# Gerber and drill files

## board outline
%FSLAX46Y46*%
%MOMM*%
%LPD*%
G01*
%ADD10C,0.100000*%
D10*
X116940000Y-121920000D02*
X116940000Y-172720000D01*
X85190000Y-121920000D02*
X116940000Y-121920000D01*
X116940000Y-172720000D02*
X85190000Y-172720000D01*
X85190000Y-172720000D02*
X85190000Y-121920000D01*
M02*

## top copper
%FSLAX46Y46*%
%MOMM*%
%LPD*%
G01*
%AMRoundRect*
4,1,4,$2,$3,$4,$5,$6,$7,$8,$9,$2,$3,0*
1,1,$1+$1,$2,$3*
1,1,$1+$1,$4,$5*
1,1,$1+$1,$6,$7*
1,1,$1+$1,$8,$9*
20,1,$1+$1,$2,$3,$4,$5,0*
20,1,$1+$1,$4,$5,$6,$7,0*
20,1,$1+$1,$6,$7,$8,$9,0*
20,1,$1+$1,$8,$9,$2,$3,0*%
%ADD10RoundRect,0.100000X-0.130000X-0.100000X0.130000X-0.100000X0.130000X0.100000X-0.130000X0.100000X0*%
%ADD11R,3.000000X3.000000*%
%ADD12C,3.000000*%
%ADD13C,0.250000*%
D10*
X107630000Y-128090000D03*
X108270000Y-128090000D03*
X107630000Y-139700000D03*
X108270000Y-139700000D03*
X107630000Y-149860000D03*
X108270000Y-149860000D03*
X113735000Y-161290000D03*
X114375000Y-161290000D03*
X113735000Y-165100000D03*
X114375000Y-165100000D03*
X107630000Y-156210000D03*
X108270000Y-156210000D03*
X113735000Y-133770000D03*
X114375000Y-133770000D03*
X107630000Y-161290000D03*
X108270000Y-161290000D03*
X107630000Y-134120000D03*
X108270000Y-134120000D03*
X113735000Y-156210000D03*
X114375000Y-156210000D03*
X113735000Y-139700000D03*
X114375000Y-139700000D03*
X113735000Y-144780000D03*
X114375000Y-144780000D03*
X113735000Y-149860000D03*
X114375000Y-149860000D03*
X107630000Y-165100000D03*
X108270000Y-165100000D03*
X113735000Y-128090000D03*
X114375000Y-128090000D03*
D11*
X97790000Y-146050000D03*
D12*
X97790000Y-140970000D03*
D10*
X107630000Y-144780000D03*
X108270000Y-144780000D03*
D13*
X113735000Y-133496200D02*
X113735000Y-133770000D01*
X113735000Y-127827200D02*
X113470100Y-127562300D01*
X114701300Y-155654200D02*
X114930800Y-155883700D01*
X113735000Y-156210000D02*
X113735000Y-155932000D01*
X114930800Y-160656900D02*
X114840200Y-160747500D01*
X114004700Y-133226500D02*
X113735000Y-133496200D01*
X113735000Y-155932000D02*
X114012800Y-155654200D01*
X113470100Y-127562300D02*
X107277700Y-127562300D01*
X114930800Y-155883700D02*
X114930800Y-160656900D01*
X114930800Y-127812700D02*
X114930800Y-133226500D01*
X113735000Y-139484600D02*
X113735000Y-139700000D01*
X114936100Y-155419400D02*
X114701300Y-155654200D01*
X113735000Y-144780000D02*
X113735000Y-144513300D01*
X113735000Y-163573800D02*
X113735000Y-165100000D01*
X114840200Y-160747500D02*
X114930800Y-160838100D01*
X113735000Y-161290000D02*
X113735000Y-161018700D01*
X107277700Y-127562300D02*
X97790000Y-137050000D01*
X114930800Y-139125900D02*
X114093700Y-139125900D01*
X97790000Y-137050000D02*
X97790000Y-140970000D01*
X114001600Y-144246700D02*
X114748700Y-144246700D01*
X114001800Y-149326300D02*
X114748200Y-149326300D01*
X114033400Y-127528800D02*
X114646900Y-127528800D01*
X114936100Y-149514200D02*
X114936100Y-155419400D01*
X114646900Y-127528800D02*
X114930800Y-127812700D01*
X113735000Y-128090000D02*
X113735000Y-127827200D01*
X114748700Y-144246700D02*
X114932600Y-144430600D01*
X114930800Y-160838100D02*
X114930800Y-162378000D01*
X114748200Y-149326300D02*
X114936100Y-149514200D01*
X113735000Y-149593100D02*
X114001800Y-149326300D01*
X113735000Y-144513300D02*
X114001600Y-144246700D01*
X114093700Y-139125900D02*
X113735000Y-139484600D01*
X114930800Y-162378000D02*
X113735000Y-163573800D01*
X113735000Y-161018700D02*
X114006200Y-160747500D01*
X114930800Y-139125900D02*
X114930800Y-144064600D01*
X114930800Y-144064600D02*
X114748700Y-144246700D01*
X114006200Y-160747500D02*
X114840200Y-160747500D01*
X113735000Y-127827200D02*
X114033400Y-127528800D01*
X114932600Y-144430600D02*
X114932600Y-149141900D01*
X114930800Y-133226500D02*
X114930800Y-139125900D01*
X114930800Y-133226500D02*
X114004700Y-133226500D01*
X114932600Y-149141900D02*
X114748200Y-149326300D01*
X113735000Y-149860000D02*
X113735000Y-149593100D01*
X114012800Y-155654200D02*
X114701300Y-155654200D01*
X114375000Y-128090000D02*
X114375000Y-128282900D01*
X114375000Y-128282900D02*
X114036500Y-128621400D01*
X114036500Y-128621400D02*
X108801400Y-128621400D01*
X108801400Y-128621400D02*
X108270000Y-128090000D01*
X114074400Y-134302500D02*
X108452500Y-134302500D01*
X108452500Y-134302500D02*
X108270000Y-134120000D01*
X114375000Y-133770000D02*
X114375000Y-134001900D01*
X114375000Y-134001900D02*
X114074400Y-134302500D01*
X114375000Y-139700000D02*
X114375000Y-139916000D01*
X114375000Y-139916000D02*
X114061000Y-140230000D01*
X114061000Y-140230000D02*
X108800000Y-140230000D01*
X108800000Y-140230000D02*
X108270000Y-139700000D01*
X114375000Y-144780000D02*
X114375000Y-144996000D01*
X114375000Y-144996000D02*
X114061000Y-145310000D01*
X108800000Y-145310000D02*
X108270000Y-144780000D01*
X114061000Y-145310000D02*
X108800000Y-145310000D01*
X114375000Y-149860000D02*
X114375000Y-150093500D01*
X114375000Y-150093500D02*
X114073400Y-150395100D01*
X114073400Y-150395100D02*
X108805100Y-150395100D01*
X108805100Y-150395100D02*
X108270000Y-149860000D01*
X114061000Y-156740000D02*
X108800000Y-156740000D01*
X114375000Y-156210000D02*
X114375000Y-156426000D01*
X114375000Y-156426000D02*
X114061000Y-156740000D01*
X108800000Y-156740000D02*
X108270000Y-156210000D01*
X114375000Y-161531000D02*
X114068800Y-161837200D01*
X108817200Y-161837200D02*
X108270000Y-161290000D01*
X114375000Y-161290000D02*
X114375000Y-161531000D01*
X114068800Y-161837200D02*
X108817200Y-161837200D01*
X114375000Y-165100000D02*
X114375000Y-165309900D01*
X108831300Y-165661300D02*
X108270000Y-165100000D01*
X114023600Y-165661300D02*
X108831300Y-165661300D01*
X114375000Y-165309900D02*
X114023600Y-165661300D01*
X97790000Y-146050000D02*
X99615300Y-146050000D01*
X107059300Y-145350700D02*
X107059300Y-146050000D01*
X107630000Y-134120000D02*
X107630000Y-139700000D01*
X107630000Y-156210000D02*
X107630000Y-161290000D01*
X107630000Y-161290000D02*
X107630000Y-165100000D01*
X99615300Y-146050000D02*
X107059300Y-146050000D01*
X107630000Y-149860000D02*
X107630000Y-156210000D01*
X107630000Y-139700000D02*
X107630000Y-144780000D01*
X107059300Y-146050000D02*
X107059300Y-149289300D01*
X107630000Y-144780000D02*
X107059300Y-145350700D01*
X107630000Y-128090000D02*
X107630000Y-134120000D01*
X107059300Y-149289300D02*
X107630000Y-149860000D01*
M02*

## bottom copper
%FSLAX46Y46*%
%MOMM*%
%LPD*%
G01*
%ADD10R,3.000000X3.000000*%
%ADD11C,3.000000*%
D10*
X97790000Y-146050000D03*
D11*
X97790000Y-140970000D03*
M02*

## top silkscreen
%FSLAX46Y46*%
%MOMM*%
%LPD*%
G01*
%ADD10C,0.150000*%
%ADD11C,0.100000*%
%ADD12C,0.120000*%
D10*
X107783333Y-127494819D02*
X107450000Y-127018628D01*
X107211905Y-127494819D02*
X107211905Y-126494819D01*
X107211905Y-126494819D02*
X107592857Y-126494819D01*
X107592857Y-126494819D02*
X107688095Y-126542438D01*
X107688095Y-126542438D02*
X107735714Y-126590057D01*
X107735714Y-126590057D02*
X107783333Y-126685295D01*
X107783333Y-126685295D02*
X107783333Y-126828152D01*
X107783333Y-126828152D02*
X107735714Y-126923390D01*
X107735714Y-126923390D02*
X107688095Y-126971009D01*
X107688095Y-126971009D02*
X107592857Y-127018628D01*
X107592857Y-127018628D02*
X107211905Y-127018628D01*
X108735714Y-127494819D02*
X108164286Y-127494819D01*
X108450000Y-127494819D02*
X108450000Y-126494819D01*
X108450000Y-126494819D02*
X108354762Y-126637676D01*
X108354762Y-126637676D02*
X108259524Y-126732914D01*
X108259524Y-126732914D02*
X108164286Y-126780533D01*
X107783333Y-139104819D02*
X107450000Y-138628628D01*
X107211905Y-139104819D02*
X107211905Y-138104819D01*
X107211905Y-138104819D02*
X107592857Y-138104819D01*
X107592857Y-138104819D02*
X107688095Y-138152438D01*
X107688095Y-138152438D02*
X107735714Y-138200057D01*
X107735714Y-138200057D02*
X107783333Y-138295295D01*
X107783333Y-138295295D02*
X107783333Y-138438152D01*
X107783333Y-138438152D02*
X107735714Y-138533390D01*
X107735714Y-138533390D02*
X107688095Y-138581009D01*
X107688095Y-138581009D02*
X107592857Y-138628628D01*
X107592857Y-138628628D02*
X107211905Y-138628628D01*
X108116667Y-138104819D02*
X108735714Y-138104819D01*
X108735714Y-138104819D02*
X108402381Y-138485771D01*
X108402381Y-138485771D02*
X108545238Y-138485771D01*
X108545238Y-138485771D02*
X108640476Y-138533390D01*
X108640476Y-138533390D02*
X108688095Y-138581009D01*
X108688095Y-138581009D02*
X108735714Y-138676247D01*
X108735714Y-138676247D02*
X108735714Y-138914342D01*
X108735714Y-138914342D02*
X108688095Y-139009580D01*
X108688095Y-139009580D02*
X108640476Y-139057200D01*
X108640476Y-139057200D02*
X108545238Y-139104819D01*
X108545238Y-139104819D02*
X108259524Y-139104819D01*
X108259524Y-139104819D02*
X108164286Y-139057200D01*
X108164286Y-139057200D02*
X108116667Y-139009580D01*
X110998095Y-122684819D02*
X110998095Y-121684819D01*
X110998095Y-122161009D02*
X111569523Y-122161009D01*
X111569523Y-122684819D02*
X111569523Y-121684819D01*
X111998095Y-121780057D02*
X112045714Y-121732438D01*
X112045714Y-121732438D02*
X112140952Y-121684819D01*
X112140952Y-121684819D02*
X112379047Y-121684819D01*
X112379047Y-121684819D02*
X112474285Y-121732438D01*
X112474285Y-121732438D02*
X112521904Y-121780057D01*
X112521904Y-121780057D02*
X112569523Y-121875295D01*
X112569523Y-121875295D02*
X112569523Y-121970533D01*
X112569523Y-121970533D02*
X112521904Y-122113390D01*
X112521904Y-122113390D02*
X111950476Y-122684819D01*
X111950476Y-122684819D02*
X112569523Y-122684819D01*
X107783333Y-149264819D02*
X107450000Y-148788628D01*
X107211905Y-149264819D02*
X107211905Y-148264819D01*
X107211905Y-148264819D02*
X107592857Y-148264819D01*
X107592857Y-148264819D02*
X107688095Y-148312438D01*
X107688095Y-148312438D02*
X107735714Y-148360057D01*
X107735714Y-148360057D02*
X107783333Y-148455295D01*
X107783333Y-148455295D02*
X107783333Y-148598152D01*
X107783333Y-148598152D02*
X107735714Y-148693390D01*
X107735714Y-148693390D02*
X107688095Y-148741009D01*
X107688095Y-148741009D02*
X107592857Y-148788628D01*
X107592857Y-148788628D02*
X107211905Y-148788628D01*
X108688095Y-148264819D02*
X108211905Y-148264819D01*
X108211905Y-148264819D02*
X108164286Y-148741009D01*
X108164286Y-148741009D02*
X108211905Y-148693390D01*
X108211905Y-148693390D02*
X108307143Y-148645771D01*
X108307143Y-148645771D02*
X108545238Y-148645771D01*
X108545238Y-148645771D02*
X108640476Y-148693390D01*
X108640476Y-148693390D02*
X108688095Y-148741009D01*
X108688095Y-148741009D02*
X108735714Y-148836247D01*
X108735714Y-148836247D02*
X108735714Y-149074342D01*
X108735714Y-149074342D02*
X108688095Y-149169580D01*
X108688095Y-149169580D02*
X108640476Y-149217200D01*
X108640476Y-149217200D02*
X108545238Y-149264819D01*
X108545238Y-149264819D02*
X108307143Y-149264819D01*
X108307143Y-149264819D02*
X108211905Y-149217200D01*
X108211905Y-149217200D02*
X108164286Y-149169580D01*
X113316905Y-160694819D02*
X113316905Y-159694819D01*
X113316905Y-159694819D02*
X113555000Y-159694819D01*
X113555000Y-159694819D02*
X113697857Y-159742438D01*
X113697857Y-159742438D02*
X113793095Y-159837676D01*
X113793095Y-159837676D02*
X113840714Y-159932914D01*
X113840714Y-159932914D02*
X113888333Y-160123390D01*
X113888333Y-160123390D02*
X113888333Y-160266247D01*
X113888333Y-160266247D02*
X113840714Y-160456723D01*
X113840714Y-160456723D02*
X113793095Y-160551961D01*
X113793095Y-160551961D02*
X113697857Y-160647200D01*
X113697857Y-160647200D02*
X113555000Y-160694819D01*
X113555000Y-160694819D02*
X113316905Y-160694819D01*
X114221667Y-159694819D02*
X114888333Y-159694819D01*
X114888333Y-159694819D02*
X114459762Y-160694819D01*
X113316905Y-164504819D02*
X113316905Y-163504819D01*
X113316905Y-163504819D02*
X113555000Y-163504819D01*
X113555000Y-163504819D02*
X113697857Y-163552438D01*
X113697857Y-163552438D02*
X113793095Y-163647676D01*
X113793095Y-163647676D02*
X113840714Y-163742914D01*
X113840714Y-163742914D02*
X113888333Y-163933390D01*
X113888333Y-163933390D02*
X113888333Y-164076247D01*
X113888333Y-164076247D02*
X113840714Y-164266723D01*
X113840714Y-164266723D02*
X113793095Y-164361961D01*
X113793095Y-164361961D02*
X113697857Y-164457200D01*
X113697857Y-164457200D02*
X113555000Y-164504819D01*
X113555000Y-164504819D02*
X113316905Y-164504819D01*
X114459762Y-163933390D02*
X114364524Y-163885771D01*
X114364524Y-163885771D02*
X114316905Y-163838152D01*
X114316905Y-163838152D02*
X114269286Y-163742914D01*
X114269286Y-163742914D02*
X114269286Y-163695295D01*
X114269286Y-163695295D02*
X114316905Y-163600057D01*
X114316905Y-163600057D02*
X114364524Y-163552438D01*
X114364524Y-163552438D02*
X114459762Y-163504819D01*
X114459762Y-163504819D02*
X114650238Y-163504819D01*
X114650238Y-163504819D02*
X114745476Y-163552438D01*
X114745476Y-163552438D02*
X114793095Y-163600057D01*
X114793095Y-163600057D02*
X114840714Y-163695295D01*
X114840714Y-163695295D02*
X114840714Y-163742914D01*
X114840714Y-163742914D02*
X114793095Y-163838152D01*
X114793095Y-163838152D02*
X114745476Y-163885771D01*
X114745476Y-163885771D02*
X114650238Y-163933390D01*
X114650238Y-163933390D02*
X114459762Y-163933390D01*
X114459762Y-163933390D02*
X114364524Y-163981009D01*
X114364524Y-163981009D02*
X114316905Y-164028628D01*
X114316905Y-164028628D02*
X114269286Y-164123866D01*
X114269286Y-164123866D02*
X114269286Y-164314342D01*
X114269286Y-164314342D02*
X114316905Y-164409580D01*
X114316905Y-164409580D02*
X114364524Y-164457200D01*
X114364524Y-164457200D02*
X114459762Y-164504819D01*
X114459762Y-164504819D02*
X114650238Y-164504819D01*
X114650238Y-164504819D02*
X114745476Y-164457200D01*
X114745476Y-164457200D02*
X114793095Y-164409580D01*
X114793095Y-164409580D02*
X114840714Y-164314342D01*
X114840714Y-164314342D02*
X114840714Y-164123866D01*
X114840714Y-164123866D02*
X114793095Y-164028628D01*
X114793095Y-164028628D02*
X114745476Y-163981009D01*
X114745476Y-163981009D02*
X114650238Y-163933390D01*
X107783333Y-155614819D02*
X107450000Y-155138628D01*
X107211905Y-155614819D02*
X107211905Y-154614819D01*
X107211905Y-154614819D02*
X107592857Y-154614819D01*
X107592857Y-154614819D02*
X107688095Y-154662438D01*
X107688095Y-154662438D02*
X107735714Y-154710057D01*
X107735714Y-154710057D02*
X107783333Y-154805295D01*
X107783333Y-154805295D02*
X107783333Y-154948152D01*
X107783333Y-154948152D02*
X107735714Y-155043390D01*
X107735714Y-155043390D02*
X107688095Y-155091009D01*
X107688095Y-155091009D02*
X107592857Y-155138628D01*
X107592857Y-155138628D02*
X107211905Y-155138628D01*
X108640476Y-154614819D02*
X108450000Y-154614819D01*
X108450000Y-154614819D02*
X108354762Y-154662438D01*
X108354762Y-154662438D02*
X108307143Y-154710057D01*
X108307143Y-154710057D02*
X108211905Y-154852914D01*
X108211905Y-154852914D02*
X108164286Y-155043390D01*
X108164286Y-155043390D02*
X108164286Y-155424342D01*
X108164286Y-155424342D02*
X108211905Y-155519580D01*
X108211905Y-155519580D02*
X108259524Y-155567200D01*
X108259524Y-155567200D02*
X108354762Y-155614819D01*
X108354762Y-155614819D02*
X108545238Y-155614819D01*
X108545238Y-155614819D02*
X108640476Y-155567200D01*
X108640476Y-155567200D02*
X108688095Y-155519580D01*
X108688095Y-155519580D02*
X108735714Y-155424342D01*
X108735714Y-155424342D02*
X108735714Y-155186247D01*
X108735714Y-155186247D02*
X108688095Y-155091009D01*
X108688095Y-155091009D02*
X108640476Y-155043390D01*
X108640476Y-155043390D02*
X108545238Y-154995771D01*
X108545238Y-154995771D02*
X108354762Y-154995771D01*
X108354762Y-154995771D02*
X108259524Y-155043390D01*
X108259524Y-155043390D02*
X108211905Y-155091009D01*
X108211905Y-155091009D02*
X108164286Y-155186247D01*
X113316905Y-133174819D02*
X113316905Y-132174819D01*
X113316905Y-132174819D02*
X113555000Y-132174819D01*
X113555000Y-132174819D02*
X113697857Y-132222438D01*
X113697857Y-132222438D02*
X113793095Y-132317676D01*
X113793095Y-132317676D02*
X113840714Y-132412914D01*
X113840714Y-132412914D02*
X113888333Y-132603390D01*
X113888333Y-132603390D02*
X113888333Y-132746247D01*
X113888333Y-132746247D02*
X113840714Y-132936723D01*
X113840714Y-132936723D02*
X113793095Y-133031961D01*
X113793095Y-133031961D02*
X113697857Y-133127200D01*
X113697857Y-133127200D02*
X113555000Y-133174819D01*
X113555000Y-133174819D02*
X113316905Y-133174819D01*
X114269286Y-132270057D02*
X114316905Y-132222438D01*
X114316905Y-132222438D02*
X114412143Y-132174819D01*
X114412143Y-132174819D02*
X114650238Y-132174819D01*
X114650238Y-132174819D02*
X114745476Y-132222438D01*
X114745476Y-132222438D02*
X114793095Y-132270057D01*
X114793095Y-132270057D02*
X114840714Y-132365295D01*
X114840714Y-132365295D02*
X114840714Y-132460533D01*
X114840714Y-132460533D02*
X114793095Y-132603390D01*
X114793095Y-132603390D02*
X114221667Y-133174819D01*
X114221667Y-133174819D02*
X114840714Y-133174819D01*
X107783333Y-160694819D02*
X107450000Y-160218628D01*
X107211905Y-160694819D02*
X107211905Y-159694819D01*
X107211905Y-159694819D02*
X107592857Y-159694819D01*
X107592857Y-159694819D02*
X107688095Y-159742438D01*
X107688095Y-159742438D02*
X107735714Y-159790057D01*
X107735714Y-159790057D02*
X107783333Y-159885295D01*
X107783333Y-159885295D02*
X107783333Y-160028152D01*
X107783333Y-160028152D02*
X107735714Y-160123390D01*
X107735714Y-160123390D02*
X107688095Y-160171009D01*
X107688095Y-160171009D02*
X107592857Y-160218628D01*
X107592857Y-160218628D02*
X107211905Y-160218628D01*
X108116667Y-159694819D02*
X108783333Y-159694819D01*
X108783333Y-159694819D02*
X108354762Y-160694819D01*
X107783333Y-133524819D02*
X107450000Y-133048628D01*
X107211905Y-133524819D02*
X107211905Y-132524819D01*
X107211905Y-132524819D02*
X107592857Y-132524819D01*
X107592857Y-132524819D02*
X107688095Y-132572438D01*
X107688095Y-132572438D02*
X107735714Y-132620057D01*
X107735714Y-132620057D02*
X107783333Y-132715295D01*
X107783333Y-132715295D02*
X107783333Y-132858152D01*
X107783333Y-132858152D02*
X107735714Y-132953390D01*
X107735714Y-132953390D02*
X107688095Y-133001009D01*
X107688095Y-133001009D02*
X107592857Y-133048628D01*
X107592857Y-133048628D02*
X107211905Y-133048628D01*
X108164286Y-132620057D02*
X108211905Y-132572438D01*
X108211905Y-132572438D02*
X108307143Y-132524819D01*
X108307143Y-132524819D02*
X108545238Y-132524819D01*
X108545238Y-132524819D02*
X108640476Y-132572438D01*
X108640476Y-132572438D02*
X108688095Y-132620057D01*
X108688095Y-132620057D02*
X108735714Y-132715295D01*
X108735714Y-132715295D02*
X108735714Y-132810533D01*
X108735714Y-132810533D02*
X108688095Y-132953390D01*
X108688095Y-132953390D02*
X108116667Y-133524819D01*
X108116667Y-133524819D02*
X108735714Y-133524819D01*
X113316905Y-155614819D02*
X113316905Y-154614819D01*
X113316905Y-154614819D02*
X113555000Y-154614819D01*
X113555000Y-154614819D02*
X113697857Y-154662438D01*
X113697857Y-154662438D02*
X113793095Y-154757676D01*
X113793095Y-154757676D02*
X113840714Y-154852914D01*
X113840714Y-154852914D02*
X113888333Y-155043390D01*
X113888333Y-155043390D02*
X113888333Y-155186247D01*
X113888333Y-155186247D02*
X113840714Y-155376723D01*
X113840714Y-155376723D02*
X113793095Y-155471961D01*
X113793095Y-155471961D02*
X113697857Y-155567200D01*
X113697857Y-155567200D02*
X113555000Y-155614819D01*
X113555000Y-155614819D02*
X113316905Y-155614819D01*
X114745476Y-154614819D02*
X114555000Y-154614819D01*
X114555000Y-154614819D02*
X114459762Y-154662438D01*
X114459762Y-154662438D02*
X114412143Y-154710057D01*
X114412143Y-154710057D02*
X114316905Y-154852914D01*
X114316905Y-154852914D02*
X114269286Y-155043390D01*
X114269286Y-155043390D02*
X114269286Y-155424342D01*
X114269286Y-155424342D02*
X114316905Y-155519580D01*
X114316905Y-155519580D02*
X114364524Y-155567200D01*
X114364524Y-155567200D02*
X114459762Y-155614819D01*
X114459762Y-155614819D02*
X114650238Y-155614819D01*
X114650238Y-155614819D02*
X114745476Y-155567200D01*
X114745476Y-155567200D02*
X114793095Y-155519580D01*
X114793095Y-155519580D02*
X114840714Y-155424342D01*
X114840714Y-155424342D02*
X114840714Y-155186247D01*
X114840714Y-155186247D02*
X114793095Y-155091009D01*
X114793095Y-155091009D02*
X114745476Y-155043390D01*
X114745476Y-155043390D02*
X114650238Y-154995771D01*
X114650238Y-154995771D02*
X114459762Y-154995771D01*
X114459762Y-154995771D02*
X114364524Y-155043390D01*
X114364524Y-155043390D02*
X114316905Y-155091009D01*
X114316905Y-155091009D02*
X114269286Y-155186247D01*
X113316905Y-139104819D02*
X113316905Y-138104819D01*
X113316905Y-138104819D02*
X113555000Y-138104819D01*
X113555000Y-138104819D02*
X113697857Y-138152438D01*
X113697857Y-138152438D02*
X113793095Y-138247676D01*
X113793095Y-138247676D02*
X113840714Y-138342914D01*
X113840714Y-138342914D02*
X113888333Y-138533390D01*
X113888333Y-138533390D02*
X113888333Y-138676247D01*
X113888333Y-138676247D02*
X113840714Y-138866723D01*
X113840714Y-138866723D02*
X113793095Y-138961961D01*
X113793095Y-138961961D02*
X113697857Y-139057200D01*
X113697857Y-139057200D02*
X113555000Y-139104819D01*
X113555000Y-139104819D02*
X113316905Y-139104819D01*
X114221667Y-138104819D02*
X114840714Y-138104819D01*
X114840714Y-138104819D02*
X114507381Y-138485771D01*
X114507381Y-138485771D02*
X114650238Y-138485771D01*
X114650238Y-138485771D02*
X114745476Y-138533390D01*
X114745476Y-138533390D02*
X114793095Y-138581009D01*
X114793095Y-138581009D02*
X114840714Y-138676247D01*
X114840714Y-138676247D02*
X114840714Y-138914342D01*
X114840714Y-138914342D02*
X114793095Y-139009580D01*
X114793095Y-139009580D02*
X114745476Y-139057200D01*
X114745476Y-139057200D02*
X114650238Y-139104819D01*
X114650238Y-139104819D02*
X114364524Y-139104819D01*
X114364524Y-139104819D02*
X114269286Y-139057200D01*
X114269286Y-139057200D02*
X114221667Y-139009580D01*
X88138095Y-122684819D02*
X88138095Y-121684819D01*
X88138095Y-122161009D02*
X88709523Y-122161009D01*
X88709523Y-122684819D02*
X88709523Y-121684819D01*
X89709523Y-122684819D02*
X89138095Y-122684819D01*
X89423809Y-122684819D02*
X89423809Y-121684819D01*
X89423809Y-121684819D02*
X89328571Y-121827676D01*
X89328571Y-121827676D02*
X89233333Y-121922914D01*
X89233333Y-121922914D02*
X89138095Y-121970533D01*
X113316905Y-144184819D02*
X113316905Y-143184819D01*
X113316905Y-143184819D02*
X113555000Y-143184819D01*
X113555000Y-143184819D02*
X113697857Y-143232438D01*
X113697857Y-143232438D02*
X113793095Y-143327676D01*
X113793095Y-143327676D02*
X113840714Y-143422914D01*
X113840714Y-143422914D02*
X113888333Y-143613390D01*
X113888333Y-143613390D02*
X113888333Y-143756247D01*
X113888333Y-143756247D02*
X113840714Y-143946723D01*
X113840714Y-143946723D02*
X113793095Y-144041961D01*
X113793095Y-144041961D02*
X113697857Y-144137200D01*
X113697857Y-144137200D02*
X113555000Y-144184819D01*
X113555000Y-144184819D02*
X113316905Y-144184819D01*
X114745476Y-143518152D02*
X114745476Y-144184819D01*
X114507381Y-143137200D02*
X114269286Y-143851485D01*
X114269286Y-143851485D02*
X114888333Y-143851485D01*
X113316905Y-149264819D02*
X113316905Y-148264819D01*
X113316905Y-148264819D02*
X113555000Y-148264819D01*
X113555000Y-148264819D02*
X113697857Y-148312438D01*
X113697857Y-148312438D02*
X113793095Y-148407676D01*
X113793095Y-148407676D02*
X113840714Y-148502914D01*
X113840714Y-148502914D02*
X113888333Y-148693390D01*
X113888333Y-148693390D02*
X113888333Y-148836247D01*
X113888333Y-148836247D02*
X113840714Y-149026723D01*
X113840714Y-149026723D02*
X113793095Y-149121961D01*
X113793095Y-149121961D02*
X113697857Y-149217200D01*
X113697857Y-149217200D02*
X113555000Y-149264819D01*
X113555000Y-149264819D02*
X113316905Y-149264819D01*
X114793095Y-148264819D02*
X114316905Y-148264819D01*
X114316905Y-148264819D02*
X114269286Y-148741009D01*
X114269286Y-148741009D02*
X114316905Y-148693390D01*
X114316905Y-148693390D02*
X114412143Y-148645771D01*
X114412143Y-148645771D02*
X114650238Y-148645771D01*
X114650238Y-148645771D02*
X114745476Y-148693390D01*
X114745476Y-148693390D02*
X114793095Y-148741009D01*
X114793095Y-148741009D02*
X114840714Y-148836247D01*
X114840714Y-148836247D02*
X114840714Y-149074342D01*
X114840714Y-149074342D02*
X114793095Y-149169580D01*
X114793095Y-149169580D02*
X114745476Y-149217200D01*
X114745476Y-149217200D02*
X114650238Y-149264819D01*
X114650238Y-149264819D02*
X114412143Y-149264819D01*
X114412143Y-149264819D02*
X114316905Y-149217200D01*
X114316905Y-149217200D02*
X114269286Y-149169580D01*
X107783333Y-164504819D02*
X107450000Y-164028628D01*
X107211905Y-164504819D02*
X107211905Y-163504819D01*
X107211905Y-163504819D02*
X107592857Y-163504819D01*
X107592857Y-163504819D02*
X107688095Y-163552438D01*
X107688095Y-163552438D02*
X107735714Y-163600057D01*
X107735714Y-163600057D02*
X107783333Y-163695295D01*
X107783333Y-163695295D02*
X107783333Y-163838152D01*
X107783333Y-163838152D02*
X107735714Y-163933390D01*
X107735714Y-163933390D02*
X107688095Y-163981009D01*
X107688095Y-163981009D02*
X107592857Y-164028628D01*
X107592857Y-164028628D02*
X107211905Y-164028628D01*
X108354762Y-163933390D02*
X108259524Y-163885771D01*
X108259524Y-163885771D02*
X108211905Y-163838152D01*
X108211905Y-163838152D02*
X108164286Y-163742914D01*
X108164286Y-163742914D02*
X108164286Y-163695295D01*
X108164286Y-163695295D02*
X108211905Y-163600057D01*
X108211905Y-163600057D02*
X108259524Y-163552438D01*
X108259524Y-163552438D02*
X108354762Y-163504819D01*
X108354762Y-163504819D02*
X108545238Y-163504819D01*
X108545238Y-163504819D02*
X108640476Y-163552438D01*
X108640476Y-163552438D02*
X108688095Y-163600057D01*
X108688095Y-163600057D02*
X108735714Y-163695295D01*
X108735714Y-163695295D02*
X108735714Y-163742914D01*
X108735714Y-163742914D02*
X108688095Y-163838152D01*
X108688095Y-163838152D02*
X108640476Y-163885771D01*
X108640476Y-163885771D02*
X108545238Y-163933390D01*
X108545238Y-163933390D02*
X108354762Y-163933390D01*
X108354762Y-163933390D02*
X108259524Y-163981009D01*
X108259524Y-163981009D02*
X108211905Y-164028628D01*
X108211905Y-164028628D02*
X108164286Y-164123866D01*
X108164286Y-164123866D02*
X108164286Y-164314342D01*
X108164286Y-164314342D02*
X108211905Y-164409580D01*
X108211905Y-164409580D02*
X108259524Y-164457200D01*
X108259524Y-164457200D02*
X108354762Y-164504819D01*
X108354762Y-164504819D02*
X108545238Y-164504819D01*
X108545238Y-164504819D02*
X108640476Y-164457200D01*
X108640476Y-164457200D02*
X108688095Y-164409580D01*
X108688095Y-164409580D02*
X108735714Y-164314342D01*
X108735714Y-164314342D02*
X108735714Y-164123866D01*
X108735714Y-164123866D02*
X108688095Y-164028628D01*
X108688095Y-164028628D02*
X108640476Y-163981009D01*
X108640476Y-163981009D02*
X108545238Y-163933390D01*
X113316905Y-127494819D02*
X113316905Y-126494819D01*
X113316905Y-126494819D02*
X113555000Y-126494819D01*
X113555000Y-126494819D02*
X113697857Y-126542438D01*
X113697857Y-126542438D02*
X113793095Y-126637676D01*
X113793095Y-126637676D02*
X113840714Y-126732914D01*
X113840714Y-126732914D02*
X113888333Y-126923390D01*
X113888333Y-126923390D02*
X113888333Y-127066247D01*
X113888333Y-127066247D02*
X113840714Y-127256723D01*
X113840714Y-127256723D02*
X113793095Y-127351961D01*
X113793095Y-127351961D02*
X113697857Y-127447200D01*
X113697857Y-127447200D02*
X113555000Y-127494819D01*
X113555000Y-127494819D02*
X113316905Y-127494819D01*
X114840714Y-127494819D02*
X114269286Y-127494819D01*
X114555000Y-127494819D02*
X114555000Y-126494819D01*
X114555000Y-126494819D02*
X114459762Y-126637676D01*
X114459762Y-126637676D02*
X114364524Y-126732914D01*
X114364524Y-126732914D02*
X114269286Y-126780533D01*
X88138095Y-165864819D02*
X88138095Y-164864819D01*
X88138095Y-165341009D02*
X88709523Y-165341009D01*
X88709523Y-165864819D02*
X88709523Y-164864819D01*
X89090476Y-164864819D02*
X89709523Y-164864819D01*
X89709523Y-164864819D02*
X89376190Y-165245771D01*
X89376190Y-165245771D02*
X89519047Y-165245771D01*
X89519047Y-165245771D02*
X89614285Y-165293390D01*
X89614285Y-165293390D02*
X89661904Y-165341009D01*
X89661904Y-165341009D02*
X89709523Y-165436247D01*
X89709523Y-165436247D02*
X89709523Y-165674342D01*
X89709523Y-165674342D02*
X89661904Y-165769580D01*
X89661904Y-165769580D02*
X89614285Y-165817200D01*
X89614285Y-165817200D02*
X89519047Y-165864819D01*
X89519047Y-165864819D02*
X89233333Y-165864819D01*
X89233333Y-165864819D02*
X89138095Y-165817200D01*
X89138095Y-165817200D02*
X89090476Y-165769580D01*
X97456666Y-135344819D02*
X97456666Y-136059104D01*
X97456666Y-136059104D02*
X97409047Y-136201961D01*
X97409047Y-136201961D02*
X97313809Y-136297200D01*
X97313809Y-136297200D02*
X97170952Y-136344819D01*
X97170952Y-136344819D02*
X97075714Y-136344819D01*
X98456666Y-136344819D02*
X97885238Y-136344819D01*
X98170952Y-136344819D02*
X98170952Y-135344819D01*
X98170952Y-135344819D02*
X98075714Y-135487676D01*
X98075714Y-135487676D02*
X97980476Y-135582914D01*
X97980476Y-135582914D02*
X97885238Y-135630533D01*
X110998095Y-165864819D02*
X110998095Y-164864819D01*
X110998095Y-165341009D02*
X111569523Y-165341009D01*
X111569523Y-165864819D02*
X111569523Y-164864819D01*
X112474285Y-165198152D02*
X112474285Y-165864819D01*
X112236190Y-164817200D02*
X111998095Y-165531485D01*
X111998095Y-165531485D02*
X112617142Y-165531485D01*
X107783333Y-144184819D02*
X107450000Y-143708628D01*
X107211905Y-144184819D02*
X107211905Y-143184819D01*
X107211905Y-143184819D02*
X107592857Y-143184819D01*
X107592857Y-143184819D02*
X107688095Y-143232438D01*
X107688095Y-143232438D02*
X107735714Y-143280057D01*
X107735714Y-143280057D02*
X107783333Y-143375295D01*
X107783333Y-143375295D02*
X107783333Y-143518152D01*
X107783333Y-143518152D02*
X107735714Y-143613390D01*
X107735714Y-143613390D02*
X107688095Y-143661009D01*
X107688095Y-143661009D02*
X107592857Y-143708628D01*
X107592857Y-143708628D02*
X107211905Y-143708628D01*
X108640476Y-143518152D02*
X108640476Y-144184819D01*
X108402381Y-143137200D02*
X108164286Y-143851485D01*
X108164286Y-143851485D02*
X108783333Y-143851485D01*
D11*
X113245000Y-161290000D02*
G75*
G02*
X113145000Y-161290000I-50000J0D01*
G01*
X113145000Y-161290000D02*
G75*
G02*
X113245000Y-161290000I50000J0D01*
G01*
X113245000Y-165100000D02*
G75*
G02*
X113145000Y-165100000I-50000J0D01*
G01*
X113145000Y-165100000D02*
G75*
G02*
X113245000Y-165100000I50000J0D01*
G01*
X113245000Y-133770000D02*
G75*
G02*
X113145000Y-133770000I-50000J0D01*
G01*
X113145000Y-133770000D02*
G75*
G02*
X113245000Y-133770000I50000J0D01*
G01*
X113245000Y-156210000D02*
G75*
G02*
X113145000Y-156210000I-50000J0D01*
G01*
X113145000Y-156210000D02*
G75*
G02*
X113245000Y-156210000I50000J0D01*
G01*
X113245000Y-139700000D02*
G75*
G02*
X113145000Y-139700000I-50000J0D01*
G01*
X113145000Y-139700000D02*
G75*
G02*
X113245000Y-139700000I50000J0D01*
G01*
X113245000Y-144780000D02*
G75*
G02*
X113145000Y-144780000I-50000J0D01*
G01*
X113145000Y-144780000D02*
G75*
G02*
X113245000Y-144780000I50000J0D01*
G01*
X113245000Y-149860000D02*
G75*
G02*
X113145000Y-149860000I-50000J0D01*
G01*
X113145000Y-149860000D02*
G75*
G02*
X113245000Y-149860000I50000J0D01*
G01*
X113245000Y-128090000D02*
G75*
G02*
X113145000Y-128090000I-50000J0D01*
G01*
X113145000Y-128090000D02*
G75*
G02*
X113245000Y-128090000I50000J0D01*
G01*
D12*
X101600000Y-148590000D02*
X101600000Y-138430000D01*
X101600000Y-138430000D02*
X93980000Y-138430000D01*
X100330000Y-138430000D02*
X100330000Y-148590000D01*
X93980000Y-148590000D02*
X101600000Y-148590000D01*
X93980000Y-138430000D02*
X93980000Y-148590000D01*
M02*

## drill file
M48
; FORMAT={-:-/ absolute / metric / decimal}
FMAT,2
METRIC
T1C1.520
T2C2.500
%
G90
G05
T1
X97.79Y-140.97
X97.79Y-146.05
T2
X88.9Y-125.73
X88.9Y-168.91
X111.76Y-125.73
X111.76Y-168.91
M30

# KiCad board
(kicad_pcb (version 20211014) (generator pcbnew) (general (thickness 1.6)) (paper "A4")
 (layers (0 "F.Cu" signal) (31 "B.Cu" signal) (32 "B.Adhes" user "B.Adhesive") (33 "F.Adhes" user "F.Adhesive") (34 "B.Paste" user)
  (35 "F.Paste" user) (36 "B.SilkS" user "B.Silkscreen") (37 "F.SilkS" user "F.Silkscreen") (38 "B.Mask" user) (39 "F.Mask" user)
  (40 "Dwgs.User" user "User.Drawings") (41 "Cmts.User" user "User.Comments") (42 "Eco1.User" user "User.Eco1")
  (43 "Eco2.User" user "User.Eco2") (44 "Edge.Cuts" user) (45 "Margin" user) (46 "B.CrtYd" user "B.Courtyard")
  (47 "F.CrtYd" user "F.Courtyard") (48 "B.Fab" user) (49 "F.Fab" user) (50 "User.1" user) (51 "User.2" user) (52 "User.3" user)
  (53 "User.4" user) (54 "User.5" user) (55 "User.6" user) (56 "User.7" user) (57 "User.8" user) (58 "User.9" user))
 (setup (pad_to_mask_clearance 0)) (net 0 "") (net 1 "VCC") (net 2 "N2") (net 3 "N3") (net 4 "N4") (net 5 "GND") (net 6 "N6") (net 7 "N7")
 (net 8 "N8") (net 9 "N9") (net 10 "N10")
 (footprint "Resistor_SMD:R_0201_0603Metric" (layer "F.Cu") (at 107.95 128.09)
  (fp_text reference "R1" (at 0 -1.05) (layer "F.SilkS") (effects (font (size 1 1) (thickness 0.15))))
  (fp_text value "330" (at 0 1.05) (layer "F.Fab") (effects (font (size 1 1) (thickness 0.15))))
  (pad "" smd roundrect (at -0.345 0) (size 0.318 0.36) (layers "F.Paste") (roundrect_rratio 0.25))
  (pad "" smd roundrect (at 0.345 0) (size 0.318 0.36) (layers "F.Paste") (roundrect_rratio 0.25))
  (pad "1" smd roundrect (at -0.32 0) (size 0.46 0.4) (layers "F.Cu" "F.Mask") (roundrect_rratio 0.25) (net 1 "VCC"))
  (pad "2" smd roundrect (at 0.32 0) (size 0.46 0.4) (layers "F.Cu" "F.Mask") (roundrect_rratio 0.25) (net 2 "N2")))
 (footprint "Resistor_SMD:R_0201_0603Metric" (layer "F.Cu") (at 107.95 139.7)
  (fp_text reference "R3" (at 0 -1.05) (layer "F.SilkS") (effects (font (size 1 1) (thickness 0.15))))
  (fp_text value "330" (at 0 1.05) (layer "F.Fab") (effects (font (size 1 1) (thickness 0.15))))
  (pad "" smd roundrect (at -0.345 0) (size 0.318 0.36) (layers "F.Paste") (roundrect_rratio 0.25))
  (pad "" smd roundrect (at 0.345 0) (size 0.318 0.36) (layers "F.Paste") (roundrect_rratio 0.25))
  (pad "1" smd roundrect (at -0.32 0) (size 0.46 0.4) (layers "F.Cu" "F.Mask") (roundrect_rratio 0.25) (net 1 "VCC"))
  (pad "2" smd roundrect (at 0.32 0) (size 0.46 0.4) (layers "F.Cu" "F.Mask") (roundrect_rratio 0.25) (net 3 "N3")))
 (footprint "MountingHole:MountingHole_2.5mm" (layer "F.Cu") (at 111.76 125.73)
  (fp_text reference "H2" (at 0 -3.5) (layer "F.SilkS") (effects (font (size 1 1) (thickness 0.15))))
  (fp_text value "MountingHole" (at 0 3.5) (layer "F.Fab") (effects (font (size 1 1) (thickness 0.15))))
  (pad "" np_thru_hole circle (at 0 0) (size 2.5 2.5) (drill 2.5) (layers *.Cu *.Mask)))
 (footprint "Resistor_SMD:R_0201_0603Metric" (layer "F.Cu") (at 107.95 149.86)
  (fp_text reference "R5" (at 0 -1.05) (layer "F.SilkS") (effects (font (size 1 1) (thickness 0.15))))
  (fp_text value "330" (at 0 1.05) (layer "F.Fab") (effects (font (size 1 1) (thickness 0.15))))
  (pad "" smd roundrect (at 0.345 0) (size 0.318 0.36) (layers "F.Paste") (roundrect_rratio 0.25))
  (pad "" smd roundrect (at -0.345 0) (size 0.318 0.36) (layers "F.Paste") (roundrect_rratio 0.25))
  (pad "1" smd roundrect (at -0.32 0) (size 0.46 0.4) (layers "F.Cu" "F.Mask") (roundrect_rratio 0.25) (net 1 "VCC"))
  (pad "2" smd roundrect (at 0.32 0) (size 0.46 0.4) (layers "F.Cu" "F.Mask") (roundrect_rratio 0.25) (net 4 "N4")))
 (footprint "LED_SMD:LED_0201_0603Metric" (layer "F.Cu") (at 114.055 161.29)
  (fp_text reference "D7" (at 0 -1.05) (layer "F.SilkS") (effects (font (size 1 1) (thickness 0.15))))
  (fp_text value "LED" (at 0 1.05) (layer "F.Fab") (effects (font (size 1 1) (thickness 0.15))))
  (fp_circle (center -0.86 0) (end -0.81 0) (layer "F.SilkS") (width 0.1) (fill none))
  (pad "" smd roundrect (at -0.345 0) (size 0.318 0.36) (layers "F.Paste") (roundrect_rratio 0.25))
  (pad "" smd roundrect (at 0.345 0) (size 0.318 0.36) (layers "F.Paste") (roundrect_rratio 0.25))
  (pad "1" smd roundrect (at -0.32 0) (size 0.46 0.4) (layers "F.Cu" "F.Mask") (roundrect_rratio 0.25) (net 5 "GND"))
  (pad "2" smd roundrect (at 0.32 0) (size 0.46 0.4) (layers "F.Cu" "F.Mask") (roundrect_rratio 0.25) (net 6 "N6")))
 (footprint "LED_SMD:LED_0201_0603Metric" (layer "F.Cu") (at 114.055 165.1)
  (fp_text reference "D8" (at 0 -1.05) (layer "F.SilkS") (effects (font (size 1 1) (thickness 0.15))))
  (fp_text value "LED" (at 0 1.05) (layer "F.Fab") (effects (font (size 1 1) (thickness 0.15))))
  (fp_circle (center -0.86 0) (end -0.81 0) (layer "F.SilkS") (width 0.1) (fill none))
  (pad "" smd roundrect (at -0.345 0) (size 0.318 0.36) (layers "F.Paste") (roundrect_rratio 0.25))
  (pad "" smd roundrect (at 0.345 0) (size 0.318 0.36) (layers "F.Paste") (roundrect_rratio 0.25))
  (pad "1" smd roundrect (at -0.32 0) (size 0.46 0.4) (layers "F.Cu" "F.Mask") (roundrect_rratio 0.25) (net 5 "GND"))
  (pad "2" smd roundrect (at 0.32 0) (size 0.46 0.4) (layers "F.Cu" "F.Mask") (roundrect_rratio 0.25) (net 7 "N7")))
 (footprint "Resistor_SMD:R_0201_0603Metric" (layer "F.Cu") (at 107.95 156.21)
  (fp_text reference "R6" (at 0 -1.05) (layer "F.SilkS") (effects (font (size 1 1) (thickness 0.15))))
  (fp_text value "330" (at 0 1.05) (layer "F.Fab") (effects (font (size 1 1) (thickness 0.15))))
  (pad "" smd roundrect (at -0.345 0) (size 0.318 0.36) (layers "F.Paste") (roundrect_rratio 0.25))
  (pad "" smd roundrect (at 0.345 0) (size 0.318 0.36) (layers "F.Paste") (roundrect_rratio 0.25))
  (pad "1" smd roundrect (at -0.32 0) (size 0.46 0.4) (layers "F.Cu" "F.Mask") (roundrect_rratio 0.25) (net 1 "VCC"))
  (pad "2" smd roundrect (at 0.32 0) (size 0.46 0.4) (layers "F.Cu" "F.Mask") (roundrect_rratio 0.25) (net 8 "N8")))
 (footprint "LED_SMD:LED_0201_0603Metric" (layer "F.Cu") (at 114.055 133.77)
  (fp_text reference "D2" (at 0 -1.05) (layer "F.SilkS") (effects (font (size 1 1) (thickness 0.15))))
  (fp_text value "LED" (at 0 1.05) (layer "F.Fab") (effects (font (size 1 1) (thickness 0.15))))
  (fp_circle (center -0.86 0) (end -0.81 0) (layer "F.SilkS") (width 0.1) (fill none))
  (pad "" smd roundrect (at 0.345 0) (size 0.318 0.36) (layers "F.Paste") (roundrect_rratio 0.25))
  (pad "" smd roundrect (at -0.345 0) (size 0.318 0.36) (layers "F.Paste") (roundrect_rratio 0.25))
  (pad "1" smd roundrect (at -0.32 0) (size 0.46 0.4) (layers "F.Cu" "F.Mask") (roundrect_rratio 0.25) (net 5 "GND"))
  (pad "2" smd roundrect (at 0.32 0) (size 0.46 0.4) (layers "F.Cu" "F.Mask") (roundrect_rratio 0.25) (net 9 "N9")))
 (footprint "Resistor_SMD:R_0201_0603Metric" (layer "F.Cu") (at 107.95 161.29)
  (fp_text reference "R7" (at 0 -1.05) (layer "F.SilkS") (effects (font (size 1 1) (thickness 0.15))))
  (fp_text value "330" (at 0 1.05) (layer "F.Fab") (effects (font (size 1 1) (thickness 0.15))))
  (pad "" smd roundrect (at -0.345 0) (size 0.318 0.36) (layers "F.Paste") (roundrect_rratio 0.25))
  (pad "" smd roundrect (at 0.345 0) (size 0.318 0.36) (layers "F.Paste") (roundrect_rratio 0.25))
  (pad "1" smd roundrect (at -0.32 0) (size 0.46 0.4) (layers "F.Cu" "F.Mask") (roundrect_rratio 0.25) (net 1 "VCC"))
  (pad "2" smd roundrect (at 0.32 0) (size 0.46 0.4) (layers "F.Cu" "F.Mask") (roundrect_rratio 0.25) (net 6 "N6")))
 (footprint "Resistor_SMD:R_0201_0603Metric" (layer "F.Cu") (at 107.95 134.12)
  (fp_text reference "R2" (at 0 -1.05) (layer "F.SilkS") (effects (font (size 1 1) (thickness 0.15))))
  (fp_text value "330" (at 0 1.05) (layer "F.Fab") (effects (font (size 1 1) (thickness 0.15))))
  (pad "" smd roundrect (at -0.345 0) (size 0.318 0.36) (layers "F.Paste") (roundrect_rratio 0.25))
  (pad "" smd roundrect (at 0.345 0) (size 0.318 0.36) (layers "F.Paste") (roundrect_rratio 0.25))
  (pad "1" smd roundrect (at -0.32 0) (size 0.46 0.4) (layers "F.Cu" "F.Mask") (roundrect_rratio 0.25) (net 1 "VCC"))
  (pad "2" smd roundrect (at 0.32 0) (size 0.46 0.4) (layers "F.Cu" "F.Mask") (roundrect_rratio 0.25) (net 9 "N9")))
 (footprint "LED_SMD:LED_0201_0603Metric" (layer "F.Cu") (at 114.055 156.21)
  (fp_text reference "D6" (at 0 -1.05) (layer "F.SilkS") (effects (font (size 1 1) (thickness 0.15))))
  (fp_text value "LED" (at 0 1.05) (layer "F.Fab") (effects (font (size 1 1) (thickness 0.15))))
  (fp_circle (center -0.86 0) (end -0.81 0) (layer "F.SilkS") (width 0.1) (fill none))
  (pad "" smd roundrect (at 0.345 0) (size 0.318 0.36) (layers "F.Paste") (roundrect_rratio 0.25))
  (pad "" smd roundrect (at -0.345 0) (size 0.318 0.36) (layers "F.Paste") (roundrect_rratio 0.25))
  (pad "1" smd roundrect (at -0.32 0) (size 0.46 0.4) (layers "F.Cu" "F.Mask") (roundrect_rratio 0.25) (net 5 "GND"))
  (pad "2" smd roundrect (at 0.32 0) (size 0.46 0.4) (layers "F.Cu" "F.Mask") (roundrect_rratio 0.25) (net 8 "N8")))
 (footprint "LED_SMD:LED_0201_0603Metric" (layer "F.Cu") (at 114.055 139.7)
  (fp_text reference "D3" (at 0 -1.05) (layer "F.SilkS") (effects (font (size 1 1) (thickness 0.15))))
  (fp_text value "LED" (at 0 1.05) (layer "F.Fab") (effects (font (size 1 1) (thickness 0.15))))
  (fp_circle (center -0.86 0) (end -0.81 0) (layer "F.SilkS") (width 0.1) (fill none))
  (pad "" smd roundrect (at -0.345 0) (size 0.318 0.36) (layers "F.Paste") (roundrect_rratio 0.25))
  (pad "" smd roundrect (at 0.345 0) (size 0.318 0.36) (layers "F.Paste") (roundrect_rratio 0.25))
  (pad "1" smd roundrect (at -0.32 0) (size 0.46 0.4) (layers "F.Cu" "F.Mask") (roundrect_rratio 0.25) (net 5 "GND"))
  (pad "2" smd roundrect (at 0.32 0) (size 0.46 0.4) (layers "F.Cu" "F.Mask") (roundrect_rratio 0.25) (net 3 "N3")))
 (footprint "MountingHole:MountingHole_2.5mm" (layer "F.Cu") (at 88.9 125.73)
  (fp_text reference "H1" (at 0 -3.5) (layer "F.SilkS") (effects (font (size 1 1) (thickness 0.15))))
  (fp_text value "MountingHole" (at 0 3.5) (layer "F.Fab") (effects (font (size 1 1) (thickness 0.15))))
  (pad "" np_thru_hole circle (at 0 0) (size 2.5 2.5) (drill 2.5) (layers *.Cu *.Mask)))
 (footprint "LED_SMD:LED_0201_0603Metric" (layer "F.Cu") (at 114.055 144.78)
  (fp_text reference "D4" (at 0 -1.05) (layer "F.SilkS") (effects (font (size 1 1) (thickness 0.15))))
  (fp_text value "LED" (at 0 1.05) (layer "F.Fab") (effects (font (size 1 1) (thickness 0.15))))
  (fp_circle (center -0.86 0) (end -0.81 0) (layer "F.SilkS") (width 0.1) (fill none))
  (pad "" smd roundrect (at 0.345 0) (size 0.318 0.36) (layers "F.Paste") (roundrect_rratio 0.25))
  (pad "" smd roundrect (at -0.345 0) (size 0.318 0.36) (layers "F.Paste") (roundrect_rratio 0.25))
  (pad "1" smd roundrect (at -0.32 0) (size 0.46 0.4) (layers "F.Cu" "F.Mask") (roundrect_rratio 0.25) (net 5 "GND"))
  (pad "2" smd roundrect (at 0.32 0) (size 0.46 0.4) (layers "F.Cu" "F.Mask") (roundrect_rratio 0.25) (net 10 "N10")))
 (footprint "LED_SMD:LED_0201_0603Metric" (layer "F.Cu") (at 114.055 149.86)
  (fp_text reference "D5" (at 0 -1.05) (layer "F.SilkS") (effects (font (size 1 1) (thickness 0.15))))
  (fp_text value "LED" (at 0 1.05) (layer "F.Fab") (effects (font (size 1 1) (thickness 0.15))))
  (fp_circle (center -0.86 0) (end -0.81 0) (layer "F.SilkS") (width 0.1) (fill none))
  (pad "" smd roundrect (at -0.345 0) (size 0.318 0.36) (layers "F.Paste") (roundrect_rratio 0.25))
  (pad "" smd roundrect (at 0.345 0) (size 0.318 0.36) (layers "F.Paste") (roundrect_rratio 0.25))
  (pad "1" smd roundrect (at -0.32 0) (size 0.46 0.4) (layers "F.Cu" "F.Mask") (roundrect_rratio 0.25) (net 5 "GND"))
  (pad "2" smd roundrect (at 0.32 0) (size 0.46 0.4) (layers "F.Cu" "F.Mask") (roundrect_rratio 0.25) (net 4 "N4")))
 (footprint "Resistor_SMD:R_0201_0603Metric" (layer "F.Cu") (at 107.95 165.1)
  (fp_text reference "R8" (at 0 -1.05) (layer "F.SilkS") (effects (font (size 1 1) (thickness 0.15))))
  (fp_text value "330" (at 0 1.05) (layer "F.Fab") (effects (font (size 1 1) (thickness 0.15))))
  (pad "" smd roundrect (at 0.345 0) (size 0.318 0.36) (layers "F.Paste") (roundrect_rratio 0.25))
  (pad "" smd roundrect (at -0.345 0) (size 0.318 0.36) (layers "F.Paste") (roundrect_rratio 0.25))
  (pad "1" smd roundrect (at -0.32 0) (size 0.46 0.4) (layers "F.Cu" "F.Mask") (roundrect_rratio 0.25) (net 1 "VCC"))
  (pad "2" smd roundrect (at 0.32 0) (size 0.46 0.4) (layers "F.Cu" "F.Mask") (roundrect_rratio 0.25) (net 7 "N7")))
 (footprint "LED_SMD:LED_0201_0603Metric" (layer "F.Cu") (at 114.055 128.09)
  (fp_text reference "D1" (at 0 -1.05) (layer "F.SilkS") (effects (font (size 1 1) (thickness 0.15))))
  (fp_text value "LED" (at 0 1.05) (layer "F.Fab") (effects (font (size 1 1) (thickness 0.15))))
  (fp_circle (center -0.86 0) (end -0.81 0) (layer "F.SilkS") (width 0.1) (fill none))
  (pad "" smd roundrect (at -0.345 0) (size 0.318 0.36) (layers "F.Paste") (roundrect_rratio 0.25))
  (pad "" smd roundrect (at 0.345 0) (size 0.318 0.36) (layers "F.Paste") (roundrect_rratio 0.25))
  (pad "1" smd roundrect (at -0.32 0) (size 0.46 0.4) (layers "F.Cu" "F.Mask") (roundrect_rratio 0.25) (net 5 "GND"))
  (pad "2" smd roundrect (at 0.32 0) (size 0.46 0.4) (layers "F.Cu" "F.Mask") (roundrect_rratio 0.25) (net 2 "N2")))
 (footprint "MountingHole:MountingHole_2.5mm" (layer "F.Cu") (at 88.9 168.91)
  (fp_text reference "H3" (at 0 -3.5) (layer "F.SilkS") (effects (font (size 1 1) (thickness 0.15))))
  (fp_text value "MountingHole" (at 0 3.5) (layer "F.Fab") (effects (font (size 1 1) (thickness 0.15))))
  (pad "" np_thru_hole circle (at 0 0) (size 2.5 2.5) (drill 2.5) (layers *.Cu *.Mask)))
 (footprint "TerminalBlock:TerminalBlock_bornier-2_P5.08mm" (layer "F.Cu") (at 97.79 146.05 90)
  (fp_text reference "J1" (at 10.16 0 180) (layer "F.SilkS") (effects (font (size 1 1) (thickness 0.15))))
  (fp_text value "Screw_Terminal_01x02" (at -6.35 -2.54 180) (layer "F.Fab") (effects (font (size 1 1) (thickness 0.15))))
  (fp_line (start -2.54 3.81) (end 7.62 3.81) (layer "F.SilkS") (width 0.12))
  (fp_line (start 7.62 3.81) (end 7.62 -3.81) (layer "F.SilkS") (width 0.12))
  (fp_line (start 7.62 2.54) (end -2.54 2.54) (layer "F.SilkS") (width 0.12))
  (fp_line (start -2.54 -3.81) (end -2.54 3.81) (layer "F.SilkS") (width 0.12))
  (fp_line (start 7.62 -3.81) (end -2.54 -3.81) (layer "F.SilkS") (width 0.12))
  (pad "1" thru_hole rect (at 0 0 90) (size 3 3) (drill 1.52) (layers *.Cu *.Mask) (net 1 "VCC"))
  (pad "2" thru_hole circle (at 5.08 0 90) (size 3 3) (drill 1.52) (layers *.Cu *.Mask) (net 5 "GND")))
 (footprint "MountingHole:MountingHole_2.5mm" (layer "F.Cu") (at 111.76 168.91)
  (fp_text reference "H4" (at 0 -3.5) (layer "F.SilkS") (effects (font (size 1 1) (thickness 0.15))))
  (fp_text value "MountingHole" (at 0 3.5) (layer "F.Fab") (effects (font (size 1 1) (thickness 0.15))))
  (pad "" np_thru_hole circle (at 0 0) (size 2.5 2.5) (drill 2.5) (layers *.Cu *.Mask)))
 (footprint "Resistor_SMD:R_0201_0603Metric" (layer "F.Cu") (at 107.95 144.78)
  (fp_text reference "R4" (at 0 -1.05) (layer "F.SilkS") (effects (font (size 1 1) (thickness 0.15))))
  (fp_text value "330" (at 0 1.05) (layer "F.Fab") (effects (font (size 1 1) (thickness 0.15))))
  (pad "" smd roundrect (at 0.345 0) (size 0.318 0.36) (layers "F.Paste") (roundrect_rratio 0.25))
  (pad "" smd roundrect (at -0.345 0) (size 0.318 0.36) (layers "F.Paste") (roundrect_rratio 0.25))
  (pad "1" smd roundrect (at -0.32 0) (size 0.46 0.4) (layers "F.Cu" "F.Mask") (roundrect_rratio 0.25) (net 1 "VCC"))
  (pad "2" smd roundrect (at 0.32 0) (size 0.46 0.4) (layers "F.Cu" "F.Mask") (roundrect_rratio 0.25) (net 10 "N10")))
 (gr_line (start 116.94 121.92) (end 116.94 172.72) (layer "Edge.Cuts") (width 0.1))
 (gr_line (start 85.19 121.92) (end 116.94 121.92) (layer "Edge.Cuts") (width 0.1))
 (gr_line (start 116.94 172.72) (end 85.19 172.72) (layer "Edge.Cuts") (width 0.1))
 (gr_line (start 85.19 172.72) (end 85.19 121.92) (layer "Edge.Cuts") (width 0.1))
 (segment (start 113.735 133.4962) (end 113.735 133.77) (width 0.25) (layer "F.Cu") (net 5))
 (segment (start 113.735 127.8272) (end 113.4701 127.5623) (width 0.25) (layer "F.Cu") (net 5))
 (segment (start 114.7013 155.6542) (end 114.9308 155.8837) (width 0.25) (layer "F.Cu") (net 5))
 (segment (start 113.735 156.21) (end 113.735 155.932) (width 0.25) (layer "F.Cu") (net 5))
 (segment (start 114.9308 160.6569) (end 114.8402 160.7475) (width 0.25) (layer "F.Cu") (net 5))
 (segment (start 114.0047 133.2265) (end 113.735 133.4962) (width 0.25) (layer "F.Cu") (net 5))
 (segment (start 113.735 155.932) (end 114.0128 155.6542) (width 0.25) (layer "F.Cu") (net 5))
 (segment (start 113.4701 127.5623) (end 107.2777 127.5623) (width 0.25) (layer "F.Cu") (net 5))
 (segment (start 114.9308 155.8837) (end 114.9308 160.6569) (width 0.25) (layer "F.Cu") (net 5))
 (segment (start 114.9308 127.8127) (end 114.9308 133.2265) (width 0.25) (layer "F.Cu") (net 5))
 (segment (start 113.735 139.4846) (end 113.735 139.7) (width 0.25) (layer "F.Cu") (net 5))
 (segment (start 114.9361 155.4194) (end 114.7013 155.6542) (width 0.25) (layer "F.Cu") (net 5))
 (segment (start 113.735 144.78) (end 113.735 144.5133) (width 0.25) (layer "F.Cu") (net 5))
 (segment (start 113.735 163.5738) (end 113.735 165.1) (width 0.25) (layer "F.Cu") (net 5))
 (segment (start 114.8402 160.7475) (end 114.9308 160.8381) (width 0.25) (layer "F.Cu") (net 5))
 (segment (start 113.735 161.29) (end 113.735 161.0187) (width 0.25) (layer "F.Cu") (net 5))
 (segment (start 107.2777 127.5623) (end 97.79 137.05) (width 0.25) (layer "F.Cu") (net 5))
 (segment (start 114.9308 139.1259) (end 114.0937 139.1259) (width 0.25) (layer "F.Cu") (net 5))
 (segment (start 97.79 137.05) (end 97.79 140.97) (width 0.25) (layer "F.Cu") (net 5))
 (segment (start 114.0016 144.2467) (end 114.7487 144.2467) (width 0.25) (layer "F.Cu") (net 5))
 (segment (start 114.0018 149.3263) (end 114.7482 149.3263) (width 0.25) (layer "F.Cu") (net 5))
 (segment (start 114.0334 127.5288) (end 114.6469 127.5288) (width 0.25) (layer "F.Cu") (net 5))
 (segment (start 114.9361 149.5142) (end 114.9361 155.4194) (width 0.25) (layer "F.Cu") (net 5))
 (segment (start 114.6469 127.5288) (end 114.9308 127.8127) (width 0.25) (layer "F.Cu") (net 5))
 (segment (start 113.735 128.09) (end 113.735 127.8272) (width 0.25) (layer "F.Cu") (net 5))
 (segment (start 114.7487 144.2467) (end 114.9326 144.4306) (width 0.25) (layer "F.Cu") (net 5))
 (segment (start 114.9308 160.8381) (end 114.9308 162.378) (width 0.25) (layer "F.Cu") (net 5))
 (segment (start 114.7482 149.3263) (end 114.9361 149.5142) (width 0.25) (layer "F.Cu") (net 5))
 (segment (start 113.735 149.5931) (end 114.0018 149.3263) (width 0.25) (layer "F.Cu") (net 5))
 (segment (start 113.735 144.5133) (end 114.0016 144.2467) (width 0.25) (layer "F.Cu") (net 5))
 (segment (start 114.0937 139.1259) (end 113.735 139.4846) (width 0.25) (layer "F.Cu") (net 5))
 (segment (start 114.9308 162.378) (end 113.735 163.5738) (width 0.25) (layer "F.Cu") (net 5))
 (segment (start 113.735 161.0187) (end 114.0062 160.7475) (width 0.25) (layer "F.Cu") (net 5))
 (segment (start 114.9308 139.1259) (end 114.9308 144.0646) (width 0.25) (layer "F.Cu") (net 5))
 (segment (start 114.9308 144.0646) (end 114.7487 144.2467) (width 0.25) (layer "F.Cu") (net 5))
 (segment (start 114.0062 160.7475) (end 114.8402 160.7475) (width 0.25) (layer "F.Cu") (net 5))
 (segment (start 113.735 127.8272) (end 114.0334 127.5288) (width 0.25) (layer "F.Cu") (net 5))
 (segment (start 114.9326 144.4306) (end 114.9326 149.1419) (width 0.25) (layer "F.Cu") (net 5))
 (segment (start 114.9308 133.2265) (end 114.9308 139.1259) (width 0.25) (layer "F.Cu") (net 5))
 (segment (start 114.9308 133.2265) (end 114.0047 133.2265) (width 0.25) (layer "F.Cu") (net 5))
 (segment (start 114.9326 149.1419) (end 114.7482 149.3263) (width 0.25) (layer "F.Cu") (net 5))
 (segment (start 113.735 149.86) (end 113.735 149.5931) (width 0.25) (layer "F.Cu") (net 5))
 (segment (start 114.0128 155.6542) (end 114.7013 155.6542) (width 0.25) (layer "F.Cu") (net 5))
 (segment (start 114.375 128.09) (end 114.375 128.2829) (width 0.25) (layer "F.Cu") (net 2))
 (segment (start 114.375 128.2829) (end 114.0365 128.6214) (width 0.25) (layer "F.Cu") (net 2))
 (segment (start 114.0365 128.6214) (end 108.8014 128.6214) (width 0.25) (layer "F.Cu") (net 2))
 (segment (start 108.8014 128.6214) (end 108.27 128.09) (width 0.25) (layer "F.Cu") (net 2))
 (segment (start 114.0744 134.3025) (end 108.4525 134.3025) (width 0.25) (layer "F.Cu") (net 9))
 (segment (start 108.4525 134.3025) (end 108.27 134.12) (width 0.25) (layer "F.Cu") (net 9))
 (segment (start 114.375 133.77) (end 114.375 134.0019) (width 0.25) (layer "F.Cu") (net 9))
 (segment (start 114.375 134.0019) (end 114.0744 134.3025) (width 0.25) (layer "F.Cu") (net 9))
 (segment (start 114.375 139.7) (end 114.375 139.916) (width 0.25) (layer "F.Cu") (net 3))
 (segment (start 114.375 139.916) (end 114.061 140.23) (width 0.25) (layer "F.Cu") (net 3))
 (segment (start 114.061 140.23) (end 108.8 140.23) (width 0.25) (layer "F.Cu") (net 3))
 (segment (start 108.8 140.23) (end 108.27 139.7) (width 0.25) (layer "F.Cu") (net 3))
 (segment (start 114.375 144.78) (end 114.375 144.996) (width 0.25) (layer "F.Cu") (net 10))
 (segment (start 114.375 144.996) (end 114.061 145.31) (width 0.25) (layer "F.Cu") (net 10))
 (segment (start 108.8 145.31) (end 108.27 144.78) (width 0.25) (layer "F.Cu") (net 10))
 (segment (start 114.061 145.31) (end 108.8 145.31) (width 0.25) (layer "F.Cu") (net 10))
 (segment (start 114.375 149.86) (end 114.375 150.0935) (width 0.25) (layer "F.Cu") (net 4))
 (segment (start 114.375 150.0935) (end 114.0734 150.3951) (width 0.25) (layer "F.Cu") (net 4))
 (segment (start 114.0734 150.3951) (end 108.8051 150.3951) (width 0.25) (layer "F.Cu") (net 4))
 (segment (start 108.8051 150.3951) (end 108.27 149.86) (width 0.25) (layer "F.Cu") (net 4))
 (segment (start 114.061 156.74) (end 108.8 156.74) (width 0.25) (layer "F.Cu") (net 8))
 (segment (start 114.375 156.21) (end 114.375 156.426) (width 0.25) (layer "F.Cu") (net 8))
 (segment (start 114.375 156.426) (end 114.061 156.74) (width 0.25) (layer "F.Cu") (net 8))
 (segment (start 108.8 156.74) (end 108.27 156.21) (width 0.25) (layer "F.Cu") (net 8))
 (segment (start 114.375 161.531) (end 114.0688 161.8372) (width 0.25) (layer "F.Cu") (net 6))
 (segment (start 108.8172 161.8372) (end 108.27 161.29) (width 0.25) (layer "F.Cu") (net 6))
 (segment (start 114.375 161.29) (end 114.375 161.531) (width 0.25) (layer "F.Cu") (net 6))
 (segment (start 114.0688 161.8372) (end 108.8172 161.8372) (width 0.25) (layer "F.Cu") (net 6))
 (segment (start 114.375 165.1) (end 114.375 165.3099) (width 0.25) (layer "F.Cu") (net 7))
 (segment (start 108.8313 165.6613) (end 108.27 165.1) (width 0.25) (layer "F.Cu") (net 7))
 (segment (start 114.0236 165.6613) (end 108.8313 165.6613) (width 0.25) (layer "F.Cu") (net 7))
 (segment (start 114.375 165.3099) (end 114.0236 165.6613) (width 0.25) (layer "F.Cu") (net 7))
 (segment (start 97.79 146.05) (end 99.6153 146.05) (width 0.25) (layer "F.Cu") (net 1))
 (segment (start 107.0593 145.3507) (end 107.0593 146.05) (width 0.25) (layer "F.Cu") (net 1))
 (segment (start 107.63 134.12) (end 107.63 139.7) (width 0.25) (layer "F.Cu") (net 1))
 (segment (start 107.63 156.21) (end 107.63 161.29) (width 0.25) (layer "F.Cu") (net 1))
 (segment (start 107.63 161.29) (end 107.63 165.1) (width 0.25) (layer "F.Cu") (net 1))
 (segment (start 99.6153 146.05) (end 107.0593 146.05) (width 0.25) (layer "F.Cu") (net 1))
 (segment (start 107.63 149.86) (end 107.63 156.21) (width 0.25) (layer "F.Cu") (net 1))
 (segment (start 107.63 139.7) (end 107.63 144.78) (width 0.25) (layer "F.Cu") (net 1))
 (segment (start 107.0593 146.05) (end 107.0593 149.2893) (width 0.25) (layer "F.Cu") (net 1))
 (segment (start 107.63 144.78) (end 107.0593 145.3507) (width 0.25) (layer "F.Cu") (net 1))
 (segment (start 107.63 128.09) (end 107.63 134.12) (width 0.25) (layer "F.Cu") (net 1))
 (segment (start 107.0593 149.2893) (end 107.63 149.86) (width 0.25) (layer "F.Cu") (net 1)))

